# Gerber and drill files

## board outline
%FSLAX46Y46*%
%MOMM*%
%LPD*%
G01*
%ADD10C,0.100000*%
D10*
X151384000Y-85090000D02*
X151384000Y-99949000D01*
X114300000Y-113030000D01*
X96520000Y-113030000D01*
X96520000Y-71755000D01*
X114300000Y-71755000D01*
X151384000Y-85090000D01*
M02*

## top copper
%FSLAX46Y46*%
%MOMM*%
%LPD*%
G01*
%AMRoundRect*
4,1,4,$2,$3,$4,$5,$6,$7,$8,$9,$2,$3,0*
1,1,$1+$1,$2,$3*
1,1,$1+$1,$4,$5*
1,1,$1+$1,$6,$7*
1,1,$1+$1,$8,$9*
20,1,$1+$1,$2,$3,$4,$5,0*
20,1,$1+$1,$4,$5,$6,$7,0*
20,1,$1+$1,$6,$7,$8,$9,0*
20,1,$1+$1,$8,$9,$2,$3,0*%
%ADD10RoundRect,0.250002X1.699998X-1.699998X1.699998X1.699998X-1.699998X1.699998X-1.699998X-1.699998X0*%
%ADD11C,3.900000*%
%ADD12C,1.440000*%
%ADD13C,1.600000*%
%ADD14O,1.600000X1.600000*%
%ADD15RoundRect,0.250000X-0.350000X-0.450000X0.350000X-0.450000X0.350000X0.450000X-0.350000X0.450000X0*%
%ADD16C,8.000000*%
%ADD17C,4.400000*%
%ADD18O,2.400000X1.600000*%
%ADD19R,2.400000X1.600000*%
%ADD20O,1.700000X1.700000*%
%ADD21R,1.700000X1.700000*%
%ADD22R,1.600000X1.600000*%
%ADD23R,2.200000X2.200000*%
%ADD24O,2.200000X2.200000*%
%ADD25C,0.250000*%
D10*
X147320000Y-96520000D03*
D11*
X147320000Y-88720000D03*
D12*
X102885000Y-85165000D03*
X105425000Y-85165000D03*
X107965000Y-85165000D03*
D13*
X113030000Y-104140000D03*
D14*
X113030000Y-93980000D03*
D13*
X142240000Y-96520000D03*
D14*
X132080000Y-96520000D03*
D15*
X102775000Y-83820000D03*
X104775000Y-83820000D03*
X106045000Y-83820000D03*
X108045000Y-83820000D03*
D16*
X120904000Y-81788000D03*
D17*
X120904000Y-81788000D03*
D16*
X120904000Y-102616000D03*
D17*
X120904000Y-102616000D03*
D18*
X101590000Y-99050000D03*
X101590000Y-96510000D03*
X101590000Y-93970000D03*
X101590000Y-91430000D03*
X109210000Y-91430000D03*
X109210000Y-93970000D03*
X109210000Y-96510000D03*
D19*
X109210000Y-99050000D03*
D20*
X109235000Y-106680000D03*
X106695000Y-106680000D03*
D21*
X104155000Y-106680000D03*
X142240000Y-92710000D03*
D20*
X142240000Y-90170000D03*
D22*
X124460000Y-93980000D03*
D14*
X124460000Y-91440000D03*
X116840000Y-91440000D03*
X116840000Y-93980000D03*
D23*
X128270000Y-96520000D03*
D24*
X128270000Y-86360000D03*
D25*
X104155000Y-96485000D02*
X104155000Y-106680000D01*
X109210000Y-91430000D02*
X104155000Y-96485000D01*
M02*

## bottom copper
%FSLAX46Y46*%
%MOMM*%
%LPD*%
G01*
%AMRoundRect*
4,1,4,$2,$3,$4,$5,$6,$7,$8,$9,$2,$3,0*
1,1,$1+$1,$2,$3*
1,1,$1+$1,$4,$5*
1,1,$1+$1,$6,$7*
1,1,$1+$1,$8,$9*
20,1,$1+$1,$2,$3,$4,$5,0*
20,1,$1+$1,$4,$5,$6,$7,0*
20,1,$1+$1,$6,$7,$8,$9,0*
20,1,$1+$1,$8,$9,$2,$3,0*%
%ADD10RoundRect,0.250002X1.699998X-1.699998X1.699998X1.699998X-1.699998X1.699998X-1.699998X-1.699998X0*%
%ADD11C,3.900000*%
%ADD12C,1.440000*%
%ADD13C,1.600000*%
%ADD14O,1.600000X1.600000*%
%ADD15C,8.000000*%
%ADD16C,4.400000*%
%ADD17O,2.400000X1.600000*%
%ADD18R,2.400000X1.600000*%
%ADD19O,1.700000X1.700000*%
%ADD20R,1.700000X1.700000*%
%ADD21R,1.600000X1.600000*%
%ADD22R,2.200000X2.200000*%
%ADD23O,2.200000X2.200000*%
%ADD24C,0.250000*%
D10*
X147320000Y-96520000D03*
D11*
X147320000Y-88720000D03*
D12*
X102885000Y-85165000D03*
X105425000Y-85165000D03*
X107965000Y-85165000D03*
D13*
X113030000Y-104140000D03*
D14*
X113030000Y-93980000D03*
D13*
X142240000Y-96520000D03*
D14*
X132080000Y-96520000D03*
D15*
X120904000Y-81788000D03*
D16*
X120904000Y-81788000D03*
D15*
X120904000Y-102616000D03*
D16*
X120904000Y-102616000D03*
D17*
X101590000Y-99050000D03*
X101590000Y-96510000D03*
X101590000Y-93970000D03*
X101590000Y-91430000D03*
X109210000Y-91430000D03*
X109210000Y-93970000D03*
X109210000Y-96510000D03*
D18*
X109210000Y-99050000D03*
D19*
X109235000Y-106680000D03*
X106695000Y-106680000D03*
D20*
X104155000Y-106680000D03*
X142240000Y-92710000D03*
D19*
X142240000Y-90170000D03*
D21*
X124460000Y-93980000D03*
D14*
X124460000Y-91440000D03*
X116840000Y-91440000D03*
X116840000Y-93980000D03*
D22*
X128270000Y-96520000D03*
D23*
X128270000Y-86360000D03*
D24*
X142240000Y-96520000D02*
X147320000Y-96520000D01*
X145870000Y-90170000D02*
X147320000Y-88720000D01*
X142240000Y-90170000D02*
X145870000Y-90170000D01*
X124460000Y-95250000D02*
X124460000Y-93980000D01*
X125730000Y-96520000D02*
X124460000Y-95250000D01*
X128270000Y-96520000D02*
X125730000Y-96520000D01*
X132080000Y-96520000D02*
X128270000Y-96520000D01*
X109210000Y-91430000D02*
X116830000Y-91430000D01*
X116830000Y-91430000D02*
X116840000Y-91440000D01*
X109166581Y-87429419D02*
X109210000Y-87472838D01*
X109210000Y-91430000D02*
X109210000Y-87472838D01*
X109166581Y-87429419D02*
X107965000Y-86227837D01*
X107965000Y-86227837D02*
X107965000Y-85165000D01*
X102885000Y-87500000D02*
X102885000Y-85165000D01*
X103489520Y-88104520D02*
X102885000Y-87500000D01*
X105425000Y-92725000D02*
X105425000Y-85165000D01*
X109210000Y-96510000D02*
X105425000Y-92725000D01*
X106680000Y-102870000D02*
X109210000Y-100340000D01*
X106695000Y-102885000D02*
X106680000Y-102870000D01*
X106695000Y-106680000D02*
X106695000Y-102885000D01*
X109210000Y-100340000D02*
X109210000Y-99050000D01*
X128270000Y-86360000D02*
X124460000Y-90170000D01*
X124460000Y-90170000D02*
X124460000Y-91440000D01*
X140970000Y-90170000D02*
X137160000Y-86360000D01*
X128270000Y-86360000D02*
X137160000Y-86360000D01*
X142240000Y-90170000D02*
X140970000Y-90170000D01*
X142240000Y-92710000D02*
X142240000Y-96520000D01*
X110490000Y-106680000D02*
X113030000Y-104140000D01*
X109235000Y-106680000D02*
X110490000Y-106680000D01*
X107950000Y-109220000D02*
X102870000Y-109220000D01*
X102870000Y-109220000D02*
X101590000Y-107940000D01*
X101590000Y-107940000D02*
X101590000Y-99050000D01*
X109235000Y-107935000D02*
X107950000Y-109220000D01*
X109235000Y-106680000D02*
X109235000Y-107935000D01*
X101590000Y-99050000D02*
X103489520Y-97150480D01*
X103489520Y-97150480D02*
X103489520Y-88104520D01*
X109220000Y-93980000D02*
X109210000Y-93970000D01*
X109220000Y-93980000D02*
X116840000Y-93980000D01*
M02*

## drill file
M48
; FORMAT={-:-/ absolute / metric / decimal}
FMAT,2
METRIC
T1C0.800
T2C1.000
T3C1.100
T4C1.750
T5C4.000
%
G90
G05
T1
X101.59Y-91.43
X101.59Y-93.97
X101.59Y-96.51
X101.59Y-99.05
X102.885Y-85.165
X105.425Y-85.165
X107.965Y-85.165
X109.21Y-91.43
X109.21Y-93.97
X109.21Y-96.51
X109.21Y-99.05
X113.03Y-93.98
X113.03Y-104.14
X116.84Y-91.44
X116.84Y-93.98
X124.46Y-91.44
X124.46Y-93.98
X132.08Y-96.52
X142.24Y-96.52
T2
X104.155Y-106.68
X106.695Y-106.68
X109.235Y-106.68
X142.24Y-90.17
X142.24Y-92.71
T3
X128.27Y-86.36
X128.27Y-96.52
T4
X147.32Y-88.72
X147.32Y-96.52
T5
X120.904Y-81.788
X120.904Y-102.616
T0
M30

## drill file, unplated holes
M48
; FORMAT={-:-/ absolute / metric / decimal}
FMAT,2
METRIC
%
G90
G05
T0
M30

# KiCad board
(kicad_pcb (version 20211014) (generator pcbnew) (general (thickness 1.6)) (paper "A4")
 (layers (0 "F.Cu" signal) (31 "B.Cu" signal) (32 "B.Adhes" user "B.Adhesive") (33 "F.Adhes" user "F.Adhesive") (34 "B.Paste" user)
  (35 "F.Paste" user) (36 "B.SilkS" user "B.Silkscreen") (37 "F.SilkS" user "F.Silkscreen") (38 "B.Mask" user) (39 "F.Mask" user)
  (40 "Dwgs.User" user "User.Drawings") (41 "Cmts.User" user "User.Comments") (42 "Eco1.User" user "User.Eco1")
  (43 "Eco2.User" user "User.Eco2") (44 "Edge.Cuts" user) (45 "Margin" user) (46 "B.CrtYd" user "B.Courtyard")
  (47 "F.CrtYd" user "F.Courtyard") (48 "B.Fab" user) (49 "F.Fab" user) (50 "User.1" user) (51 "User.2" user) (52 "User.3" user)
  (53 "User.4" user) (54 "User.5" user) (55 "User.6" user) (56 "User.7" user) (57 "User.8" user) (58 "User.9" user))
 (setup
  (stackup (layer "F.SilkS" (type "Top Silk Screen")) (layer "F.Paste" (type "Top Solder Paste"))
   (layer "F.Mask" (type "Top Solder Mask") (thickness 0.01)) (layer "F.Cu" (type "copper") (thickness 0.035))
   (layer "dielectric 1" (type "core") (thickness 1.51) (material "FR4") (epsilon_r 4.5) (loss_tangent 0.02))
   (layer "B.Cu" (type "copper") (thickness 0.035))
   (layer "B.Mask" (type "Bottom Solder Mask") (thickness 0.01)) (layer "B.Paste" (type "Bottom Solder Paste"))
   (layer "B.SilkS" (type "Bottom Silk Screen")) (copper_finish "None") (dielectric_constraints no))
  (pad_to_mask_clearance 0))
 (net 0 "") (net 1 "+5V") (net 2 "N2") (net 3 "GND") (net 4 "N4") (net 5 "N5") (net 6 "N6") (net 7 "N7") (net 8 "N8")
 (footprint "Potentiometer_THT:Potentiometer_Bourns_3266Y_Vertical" (layer "F.Cu") (at 102.885 85.165 180)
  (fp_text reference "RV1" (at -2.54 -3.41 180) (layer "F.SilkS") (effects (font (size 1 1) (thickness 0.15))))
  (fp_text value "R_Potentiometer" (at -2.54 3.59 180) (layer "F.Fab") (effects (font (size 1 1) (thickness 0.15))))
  (pad "1" thru_hole circle (at 0 0 180) (size 1.44 1.44) (drill 0.8) (layers *.Cu *.Mask) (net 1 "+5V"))
  (pad "2" thru_hole circle (at -2.54 0 180) (size 1.44 1.44) (drill 0.8) (layers *.Cu *.Mask) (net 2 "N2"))
  (pad "3" thru_hole circle (at -5.08 0 180) (size 1.44 1.44) (drill 0.8) (layers *.Cu *.Mask) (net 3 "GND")))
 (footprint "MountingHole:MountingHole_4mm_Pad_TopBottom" (layer "F.Cu") (at 120.904 102.616)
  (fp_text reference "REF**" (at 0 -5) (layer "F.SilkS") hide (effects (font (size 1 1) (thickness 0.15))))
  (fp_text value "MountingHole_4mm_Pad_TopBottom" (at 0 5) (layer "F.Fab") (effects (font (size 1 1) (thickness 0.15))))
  (pad "1" thru_hole circle (at 0 0) (size 4.4 4.4) (drill 4) (layers *.Cu *.Mask))
  (pad "1" connect circle (at 0 0) (size 8 8) (layers "F.Cu" "F.Mask"))
  (pad "1" connect circle (at 0 0) (size 8 8) (layers "B.Cu" "B.Mask")))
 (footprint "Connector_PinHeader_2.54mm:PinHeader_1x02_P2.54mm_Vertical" (layer "F.Cu") (at 142.24 92.71 180)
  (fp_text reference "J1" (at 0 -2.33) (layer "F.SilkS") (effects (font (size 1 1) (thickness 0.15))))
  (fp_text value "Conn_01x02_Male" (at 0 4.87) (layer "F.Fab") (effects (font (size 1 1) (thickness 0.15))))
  (pad "1" thru_hole rect (at 0 0 180) (size 1.7 1.7) (drill 1) (layers *.Cu *.Mask) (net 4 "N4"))
  (pad "2" thru_hole oval (at 0 2.54 180) (size 1.7 1.7) (drill 1) (layers *.Cu *.Mask) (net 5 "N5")))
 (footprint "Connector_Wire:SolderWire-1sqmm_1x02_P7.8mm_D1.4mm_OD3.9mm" (layer "F.Cu") (at 147.32 96.52 90)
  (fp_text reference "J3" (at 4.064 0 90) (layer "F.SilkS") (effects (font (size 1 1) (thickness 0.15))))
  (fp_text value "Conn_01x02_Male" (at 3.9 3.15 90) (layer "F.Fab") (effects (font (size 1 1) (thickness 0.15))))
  (pad "1" thru_hole roundrect (at 0 0 90) (size 3.9 3.9) (drill 1.75) (layers *.Cu *.Mask) (roundrect_rratio 0.064103) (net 4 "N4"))
  (pad "2" thru_hole circle (at 7.8 0 90) (size 3.9 3.9) (drill 1.75) (layers *.Cu *.Mask) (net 5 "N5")))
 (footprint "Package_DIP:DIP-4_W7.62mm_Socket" (layer "F.Cu") (at 124.46 93.98 180)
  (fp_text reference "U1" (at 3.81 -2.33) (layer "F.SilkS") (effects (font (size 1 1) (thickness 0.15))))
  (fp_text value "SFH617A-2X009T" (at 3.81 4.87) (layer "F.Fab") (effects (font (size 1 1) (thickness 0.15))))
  (pad "1" thru_hole rect (at 0 0 180) (size 1.6 1.6) (drill 0.8) (layers *.Cu *.Mask) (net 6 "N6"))
  (pad "2" thru_hole oval (at 0 2.54 180) (size 1.6 1.6) (drill 0.8) (layers *.Cu *.Mask) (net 5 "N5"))
  (pad "3" thru_hole oval (at 7.62 2.54 180) (size 1.6 1.6) (drill 0.8) (layers *.Cu *.Mask) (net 3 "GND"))
  (pad "4" thru_hole oval (at 7.62 0 180) (size 1.6 1.6) (drill 0.8) (layers *.Cu *.Mask) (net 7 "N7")))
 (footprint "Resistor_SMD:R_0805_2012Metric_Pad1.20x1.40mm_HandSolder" (layer "F.Cu") (at 103.775 83.82)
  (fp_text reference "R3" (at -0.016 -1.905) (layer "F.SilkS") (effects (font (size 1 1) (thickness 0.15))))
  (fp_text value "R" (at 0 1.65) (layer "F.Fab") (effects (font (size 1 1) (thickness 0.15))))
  (pad "1" smd roundrect (at -1 0) (size 1.2 1.4) (layers "F.Cu" "F.Paste" "F.Mask") (roundrect_rratio 0.2083333333) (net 1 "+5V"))
  (pad "2" smd roundrect (at 1 0) (size 1.2 1.4) (layers "F.Cu" "F.Paste" "F.Mask") (roundrect_rratio 0.2083333333) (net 2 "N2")))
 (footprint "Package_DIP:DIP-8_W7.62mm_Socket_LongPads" (layer "F.Cu") (at 109.21 99.05 180)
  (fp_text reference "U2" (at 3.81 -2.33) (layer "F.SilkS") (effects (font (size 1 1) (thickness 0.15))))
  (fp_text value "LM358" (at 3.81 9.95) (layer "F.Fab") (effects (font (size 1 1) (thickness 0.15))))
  (pad "1" thru_hole rect (at 0 0 180) (size 2.4 1.6) (drill 0.8) (layers *.Cu *.Mask) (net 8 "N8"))
  (pad "2" thru_hole oval (at 0 2.54 180) (size 2.4 1.6) (drill 0.8) (layers *.Cu *.Mask) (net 2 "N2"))
  (pad "3" thru_hole oval (at 0 5.08 180) (size 2.4 1.6) (drill 0.8) (layers *.Cu *.Mask) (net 7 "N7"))
  (pad "4" thru_hole oval (at 0 7.62 180) (size 2.4 1.6) (drill 0.8) (layers *.Cu *.Mask) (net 3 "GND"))
  (pad "5" thru_hole oval (at 7.62 7.62 180) (size 2.4 1.6) (drill 0.8) (layers *.Cu *.Mask))
  (pad "6" thru_hole oval (at 7.62 5.08 180) (size 2.4 1.6) (drill 0.8) (layers *.Cu *.Mask))
  (pad "7" thru_hole oval (at 7.62 2.54 180) (size 2.4 1.6) (drill 0.8) (layers *.Cu *.Mask))
  (pad "8" thru_hole oval (at 7.62 0 180) (size 2.4 1.6) (drill 0.8) (layers *.Cu *.Mask) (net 1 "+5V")))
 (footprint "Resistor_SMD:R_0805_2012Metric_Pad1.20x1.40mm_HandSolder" (layer "F.Cu") (at 107.045 83.82)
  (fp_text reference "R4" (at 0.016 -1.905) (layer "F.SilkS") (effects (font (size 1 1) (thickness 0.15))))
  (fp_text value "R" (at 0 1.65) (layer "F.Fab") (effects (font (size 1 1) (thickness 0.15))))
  (pad "1" smd roundrect (at -1 0) (size 1.2 1.4) (layers "F.Cu" "F.Paste" "F.Mask") (roundrect_rratio 0.2083333333) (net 2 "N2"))
  (pad "2" smd roundrect (at 1 0) (size 1.2 1.4) (layers "F.Cu" "F.Paste" "F.Mask") (roundrect_rratio 0.2083333333) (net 3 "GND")))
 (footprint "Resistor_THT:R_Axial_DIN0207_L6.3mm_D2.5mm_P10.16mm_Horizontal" (layer "F.Cu") (at 142.24 96.52 180)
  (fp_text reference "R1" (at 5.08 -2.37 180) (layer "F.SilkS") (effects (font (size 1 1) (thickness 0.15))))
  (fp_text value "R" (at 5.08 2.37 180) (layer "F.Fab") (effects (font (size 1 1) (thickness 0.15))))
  (pad "1" thru_hole circle (at 0 0 180) (size 1.6 1.6) (drill 0.8) (layers *.Cu *.Mask) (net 4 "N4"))
  (pad "2" thru_hole oval (at 10.16 0 180) (size 1.6 1.6) (drill 0.8) (layers *.Cu *.Mask) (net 6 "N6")))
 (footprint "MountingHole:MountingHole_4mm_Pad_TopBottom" (layer "F.Cu") (at 120.904 81.788)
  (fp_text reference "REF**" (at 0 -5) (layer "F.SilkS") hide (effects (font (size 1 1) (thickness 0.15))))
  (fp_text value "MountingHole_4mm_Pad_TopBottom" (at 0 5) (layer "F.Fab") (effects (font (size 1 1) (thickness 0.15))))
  (pad "1" thru_hole circle (at 0 0) (size 4.4 4.4) (drill 4) (layers *.Cu *.Mask))
  (pad "1" connect circle (at 0 0) (size 8 8) (layers "F.Cu" "F.Mask"))
  (pad "1" connect circle (at 0 0) (size 8 8) (layers "B.Cu" "B.Mask")))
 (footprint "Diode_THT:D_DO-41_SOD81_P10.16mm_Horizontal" (layer "F.Cu") (at 128.27 96.52 90)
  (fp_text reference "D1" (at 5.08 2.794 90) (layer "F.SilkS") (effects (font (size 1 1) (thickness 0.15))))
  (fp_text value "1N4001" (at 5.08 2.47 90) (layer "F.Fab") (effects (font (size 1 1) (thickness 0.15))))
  (pad "1" thru_hole rect (at 0 0 90) (size 2.2 2.2) (drill 1.1) (layers *.Cu *.Mask) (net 6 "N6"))
  (pad "2" thru_hole oval (at 10.16 0 90) (size 2.2 2.2) (drill 1.1) (layers *.Cu *.Mask) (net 5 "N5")))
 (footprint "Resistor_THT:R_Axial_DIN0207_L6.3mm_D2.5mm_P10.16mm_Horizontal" (layer "F.Cu") (at 113.03 104.14 90)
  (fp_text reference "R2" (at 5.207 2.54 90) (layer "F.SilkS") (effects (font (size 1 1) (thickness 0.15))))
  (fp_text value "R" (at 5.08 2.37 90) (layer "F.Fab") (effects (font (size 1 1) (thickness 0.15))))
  (pad "1" thru_hole circle (at 0 0 90) (size 1.6 1.6) (drill 0.8) (layers *.Cu *.Mask) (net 1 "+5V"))
  (pad "2" thru_hole oval (at 10.16 0 90) (size 1.6 1.6) (drill 0.8) (layers *.Cu *.Mask) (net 7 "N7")))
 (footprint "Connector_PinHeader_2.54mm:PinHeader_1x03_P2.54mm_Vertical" (layer "F.Cu") (at 104.155 106.68 90)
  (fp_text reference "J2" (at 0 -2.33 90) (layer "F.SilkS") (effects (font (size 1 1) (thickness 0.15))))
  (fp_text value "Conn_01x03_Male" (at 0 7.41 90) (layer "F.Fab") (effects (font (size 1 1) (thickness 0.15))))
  (pad "1" thru_hole rect (at 0 0 90) (size 1.7 1.7) (drill 1) (layers *.Cu *.Mask) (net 3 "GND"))
  (pad "2" thru_hole oval (at 0 2.54 90) (size 1.7 1.7) (drill 1) (layers *.Cu *.Mask) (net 8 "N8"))
  (pad "3" thru_hole oval (at 0 5.08 90) (size 1.7 1.7) (drill 1) (layers *.Cu *.Mask) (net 1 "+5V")))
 (gr_poly
  (pts (xy 151.384 85.09) (xy 151.384 99.949) (xy 114.3 113.03) (xy 96.52 113.03) (xy 96.52 71.755) (xy 114.3 71.755)) (layer "Edge.Cuts")
  (width 0.1) (fill none))
 (segment (start 128.27 96.52) (end 125.73 96.52) (width 0.25) (layer "B.Cu") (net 6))
 (segment (start 125.73 96.52) (end 124.46 95.25) (width 0.25) (layer "B.Cu") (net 6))
 (segment (start 124.46 95.25) (end 124.46 93.98) (width 0.25) (layer "B.Cu") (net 6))
 (segment (start 132.08 96.52) (end 128.27 96.52) (width 0.25) (layer "B.Cu") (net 6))
 (segment (start 128.27 86.36) (end 124.46 90.17) (width 0.25) (layer "B.Cu") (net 5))
 (segment (start 142.24 90.17) (end 140.97 90.17) (width 0.25) (layer "B.Cu") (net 5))
 (segment (start 128.27 86.36) (end 137.16 86.36) (width 0.25) (layer "B.Cu") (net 5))
 (segment (start 145.87 90.17) (end 147.32 88.72) (width 0.25) (layer "B.Cu") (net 5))
 (segment (start 124.46 90.17) (end 124.46 91.44) (width 0.25) (layer "B.Cu") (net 5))
 (segment (start 140.97 90.17) (end 137.16 86.36) (width 0.25) (layer "B.Cu") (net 5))
 (segment (start 142.24 90.17) (end 145.87 90.17) (width 0.25) (layer "B.Cu") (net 5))
 (segment (start 142.24 96.52) (end 147.32 96.52) (width 0.25) (layer "B.Cu") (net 4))
 (segment (start 142.24 92.71) (end 142.24 96.52) (width 0.25) (layer "B.Cu") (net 4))
 (segment (start 104.155 96.485) (end 104.155 106.68) (width 0.25) (layer "F.Cu") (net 3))
 (segment (start 109.21 91.43) (end 104.155 96.485) (width 0.25) (layer "F.Cu") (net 3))
 (segment (start 107.965 86.227837) (end 107.965 85.165) (width 0.25) (layer "B.Cu") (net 3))
 (segment (start 116.83 91.43) (end 116.84 91.44) (width 0.25) (layer "B.Cu") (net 3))
 (segment (start 109.166581 87.429419) (end 107.965 86.227837) (width 0.25) (layer "B.Cu") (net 3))
 (segment (start 109.166581 87.429419) (end 109.21 87.472838) (width 0.25) (layer "B.Cu") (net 3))
 (segment (start 109.21 91.43) (end 109.21 87.472838) (width 0.25) (layer "B.Cu") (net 3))
 (segment (start 109.21 91.43) (end 116.83 91.43) (width 0.25) (layer "B.Cu") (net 3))
 (segment (start 103.48952 88.10452) (end 102.885 87.5) (width 0.25) (layer "B.Cu") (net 1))
 (segment (start 109.235 106.68) (end 109.235 107.935) (width 0.25) (layer "B.Cu") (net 1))
 (segment (start 102.87 109.22) (end 101.59 107.94) (width 0.25) (layer "B.Cu") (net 1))
 (segment (start 109.235 106.68) (end 110.49 106.68) (width 0.25) (layer "B.Cu") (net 1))
 (segment (start 110.49 106.68) (end 113.03 104.14) (width 0.25) (layer "B.Cu") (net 1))
 (segment (start 101.59 107.94) (end 101.59 99.05) (width 0.25) (layer "B.Cu") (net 1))
 (segment (start 109.235 107.935) (end 107.95 109.22) (width 0.25) (layer "B.Cu") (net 1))
 (segment (start 107.95 109.22) (end 102.87 109.22) (width 0.25) (layer "B.Cu") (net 1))
 (segment (start 103.48952 97.15048) (end 103.48952 88.10452) (width 0.25) (layer "B.Cu") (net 1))
 (segment (start 101.59 99.05) (end 103.48952 97.15048) (width 0.25) (layer "B.Cu") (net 1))
 (segment (start 102.885 87.5) (end 102.885 85.165) (width 0.25) (layer "B.Cu") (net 1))
 (segment (start 109.22 93.98) (end 109.21 93.97) (width 0.25) (layer "B.Cu") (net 7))
 (segment (start 109.22 93.98) (end 116.84 93.98) (width 0.25) (layer "B.Cu") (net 7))
 (segment (start 109.21 96.51) (end 105.425 92.725) (width 0.25) (layer "B.Cu") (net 2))
 (segment (start 105.425 92.725) (end 105.425 85.165) (width 0.25) (layer "B.Cu") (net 2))
 (segment (start 106.68 102.87) (end 109.21 100.34) (width 0.25) (layer "B.Cu") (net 8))
 (segment (start 109.21 100.34) (end 109.21 99.05) (width 0.25) (layer "B.Cu") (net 8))
 (segment (start 106.695 106.68) (end 106.695 102.885) (width 0.25) (layer "B.Cu") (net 8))
 (segment (start 106.695 102.885) (end 106.68 102.87) (width 0.25) (layer "B.Cu") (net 8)))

